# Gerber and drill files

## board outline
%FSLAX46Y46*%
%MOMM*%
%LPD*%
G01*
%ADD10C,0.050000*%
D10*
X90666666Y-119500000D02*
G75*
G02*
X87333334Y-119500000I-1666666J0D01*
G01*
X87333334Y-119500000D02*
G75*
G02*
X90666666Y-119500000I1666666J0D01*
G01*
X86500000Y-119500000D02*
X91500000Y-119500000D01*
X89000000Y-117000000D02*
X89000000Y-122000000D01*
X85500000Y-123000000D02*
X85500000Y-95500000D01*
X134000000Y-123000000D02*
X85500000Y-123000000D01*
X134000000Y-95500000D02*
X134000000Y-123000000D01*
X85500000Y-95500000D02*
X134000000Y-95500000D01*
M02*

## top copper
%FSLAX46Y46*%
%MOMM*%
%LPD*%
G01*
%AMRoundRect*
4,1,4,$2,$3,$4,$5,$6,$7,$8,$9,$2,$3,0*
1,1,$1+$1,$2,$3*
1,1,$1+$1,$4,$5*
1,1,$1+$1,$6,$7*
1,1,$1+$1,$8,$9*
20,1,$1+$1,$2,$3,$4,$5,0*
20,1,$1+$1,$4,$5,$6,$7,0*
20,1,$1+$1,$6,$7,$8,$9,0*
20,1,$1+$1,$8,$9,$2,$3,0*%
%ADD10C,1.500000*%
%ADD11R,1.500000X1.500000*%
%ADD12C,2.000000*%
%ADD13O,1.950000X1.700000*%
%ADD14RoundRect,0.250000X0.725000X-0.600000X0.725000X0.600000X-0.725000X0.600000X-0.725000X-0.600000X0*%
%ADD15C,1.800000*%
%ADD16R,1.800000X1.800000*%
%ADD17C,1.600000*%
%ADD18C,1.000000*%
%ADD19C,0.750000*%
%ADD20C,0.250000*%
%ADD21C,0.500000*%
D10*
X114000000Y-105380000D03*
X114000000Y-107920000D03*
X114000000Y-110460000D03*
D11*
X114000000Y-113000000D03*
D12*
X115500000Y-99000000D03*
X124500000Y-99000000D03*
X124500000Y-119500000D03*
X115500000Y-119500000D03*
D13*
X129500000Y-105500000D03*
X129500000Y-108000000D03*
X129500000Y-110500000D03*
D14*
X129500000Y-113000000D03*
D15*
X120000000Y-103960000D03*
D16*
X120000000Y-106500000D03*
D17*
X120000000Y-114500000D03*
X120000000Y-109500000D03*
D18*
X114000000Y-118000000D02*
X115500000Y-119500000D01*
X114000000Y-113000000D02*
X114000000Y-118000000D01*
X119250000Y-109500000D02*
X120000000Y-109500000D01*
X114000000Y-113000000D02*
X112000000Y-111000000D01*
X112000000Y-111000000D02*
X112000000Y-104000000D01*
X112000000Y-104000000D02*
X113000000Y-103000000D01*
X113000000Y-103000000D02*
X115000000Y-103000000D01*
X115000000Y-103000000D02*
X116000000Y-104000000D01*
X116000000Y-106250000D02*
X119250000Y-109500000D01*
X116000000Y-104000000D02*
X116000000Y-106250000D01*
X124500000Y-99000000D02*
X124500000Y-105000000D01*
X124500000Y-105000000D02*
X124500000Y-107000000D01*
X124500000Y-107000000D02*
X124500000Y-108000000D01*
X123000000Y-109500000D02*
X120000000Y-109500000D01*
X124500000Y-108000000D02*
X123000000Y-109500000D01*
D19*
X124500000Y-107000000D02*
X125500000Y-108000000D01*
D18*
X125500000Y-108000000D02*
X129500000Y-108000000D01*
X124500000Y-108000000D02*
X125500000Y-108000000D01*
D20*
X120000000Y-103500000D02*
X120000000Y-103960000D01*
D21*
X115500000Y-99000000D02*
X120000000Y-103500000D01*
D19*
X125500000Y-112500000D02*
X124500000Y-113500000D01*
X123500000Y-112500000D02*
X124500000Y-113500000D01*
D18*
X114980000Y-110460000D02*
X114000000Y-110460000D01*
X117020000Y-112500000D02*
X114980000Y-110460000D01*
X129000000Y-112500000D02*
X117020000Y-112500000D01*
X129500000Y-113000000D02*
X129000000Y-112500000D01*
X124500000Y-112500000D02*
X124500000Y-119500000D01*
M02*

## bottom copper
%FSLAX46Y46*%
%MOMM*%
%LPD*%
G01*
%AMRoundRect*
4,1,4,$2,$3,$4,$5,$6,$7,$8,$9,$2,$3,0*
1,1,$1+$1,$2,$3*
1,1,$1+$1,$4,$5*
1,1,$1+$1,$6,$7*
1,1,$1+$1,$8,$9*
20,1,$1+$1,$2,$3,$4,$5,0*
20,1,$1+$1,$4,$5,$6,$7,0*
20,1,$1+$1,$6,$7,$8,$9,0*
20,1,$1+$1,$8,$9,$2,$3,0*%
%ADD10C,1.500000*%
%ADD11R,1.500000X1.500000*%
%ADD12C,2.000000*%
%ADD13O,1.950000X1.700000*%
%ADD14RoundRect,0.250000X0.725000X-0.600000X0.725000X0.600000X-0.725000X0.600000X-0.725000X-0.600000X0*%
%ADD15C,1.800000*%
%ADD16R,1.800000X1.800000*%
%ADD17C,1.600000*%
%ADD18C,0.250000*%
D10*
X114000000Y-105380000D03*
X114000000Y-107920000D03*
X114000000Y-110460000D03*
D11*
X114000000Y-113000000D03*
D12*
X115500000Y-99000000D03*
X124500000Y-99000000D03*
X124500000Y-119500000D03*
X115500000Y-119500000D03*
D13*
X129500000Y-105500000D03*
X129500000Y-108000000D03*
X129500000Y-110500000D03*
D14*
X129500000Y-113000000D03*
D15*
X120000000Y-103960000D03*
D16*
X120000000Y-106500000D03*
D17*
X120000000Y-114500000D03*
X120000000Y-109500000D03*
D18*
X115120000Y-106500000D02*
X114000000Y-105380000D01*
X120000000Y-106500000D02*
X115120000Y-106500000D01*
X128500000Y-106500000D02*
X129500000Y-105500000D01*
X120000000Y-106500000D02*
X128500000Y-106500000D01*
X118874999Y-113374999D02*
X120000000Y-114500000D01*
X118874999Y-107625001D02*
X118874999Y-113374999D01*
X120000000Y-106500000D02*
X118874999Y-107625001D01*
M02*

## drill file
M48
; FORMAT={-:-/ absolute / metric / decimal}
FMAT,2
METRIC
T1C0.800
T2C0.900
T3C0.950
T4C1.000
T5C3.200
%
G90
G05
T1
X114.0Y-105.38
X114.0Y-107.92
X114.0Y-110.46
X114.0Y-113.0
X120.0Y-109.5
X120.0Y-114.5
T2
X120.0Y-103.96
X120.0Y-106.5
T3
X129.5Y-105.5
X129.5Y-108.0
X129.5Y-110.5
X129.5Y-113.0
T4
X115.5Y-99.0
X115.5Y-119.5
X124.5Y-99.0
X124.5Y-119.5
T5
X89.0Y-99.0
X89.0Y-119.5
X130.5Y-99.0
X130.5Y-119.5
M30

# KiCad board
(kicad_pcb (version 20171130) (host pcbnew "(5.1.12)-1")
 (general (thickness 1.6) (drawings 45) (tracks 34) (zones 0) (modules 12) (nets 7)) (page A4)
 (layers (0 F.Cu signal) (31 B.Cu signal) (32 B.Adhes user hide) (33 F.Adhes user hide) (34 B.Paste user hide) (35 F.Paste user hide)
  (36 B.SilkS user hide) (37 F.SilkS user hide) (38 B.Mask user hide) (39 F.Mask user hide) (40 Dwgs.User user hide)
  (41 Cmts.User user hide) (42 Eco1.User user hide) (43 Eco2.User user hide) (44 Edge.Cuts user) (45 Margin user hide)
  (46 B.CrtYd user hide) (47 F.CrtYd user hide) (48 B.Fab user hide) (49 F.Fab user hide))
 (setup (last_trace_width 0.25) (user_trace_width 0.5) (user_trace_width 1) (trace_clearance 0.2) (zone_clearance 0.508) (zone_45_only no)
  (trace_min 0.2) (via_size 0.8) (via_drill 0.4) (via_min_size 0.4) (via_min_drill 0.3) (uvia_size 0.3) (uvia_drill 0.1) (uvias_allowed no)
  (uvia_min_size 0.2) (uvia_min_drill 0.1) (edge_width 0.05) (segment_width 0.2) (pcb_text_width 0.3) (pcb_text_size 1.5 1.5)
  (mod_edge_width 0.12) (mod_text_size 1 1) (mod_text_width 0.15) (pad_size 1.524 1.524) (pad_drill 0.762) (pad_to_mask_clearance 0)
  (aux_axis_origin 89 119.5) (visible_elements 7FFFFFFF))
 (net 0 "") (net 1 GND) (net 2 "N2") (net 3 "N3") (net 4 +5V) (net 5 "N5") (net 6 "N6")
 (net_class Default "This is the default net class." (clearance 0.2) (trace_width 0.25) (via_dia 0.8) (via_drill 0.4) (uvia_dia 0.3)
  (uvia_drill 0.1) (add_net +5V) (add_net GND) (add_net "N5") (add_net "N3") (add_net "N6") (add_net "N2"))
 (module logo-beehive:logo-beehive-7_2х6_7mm (layer F.Cu) (at 98 119)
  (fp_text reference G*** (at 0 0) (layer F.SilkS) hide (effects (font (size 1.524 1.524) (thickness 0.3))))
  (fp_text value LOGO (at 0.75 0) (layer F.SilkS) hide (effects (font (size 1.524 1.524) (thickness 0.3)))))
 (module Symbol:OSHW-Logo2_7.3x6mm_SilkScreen (layer F.Cu) (at 106.5 119.5)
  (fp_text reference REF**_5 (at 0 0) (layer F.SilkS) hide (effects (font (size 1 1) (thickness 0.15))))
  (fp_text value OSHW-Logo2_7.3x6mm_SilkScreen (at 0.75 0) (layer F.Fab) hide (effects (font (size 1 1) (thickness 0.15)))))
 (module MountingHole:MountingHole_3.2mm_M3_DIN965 (layer F.Cu) (at 89 119.5 180)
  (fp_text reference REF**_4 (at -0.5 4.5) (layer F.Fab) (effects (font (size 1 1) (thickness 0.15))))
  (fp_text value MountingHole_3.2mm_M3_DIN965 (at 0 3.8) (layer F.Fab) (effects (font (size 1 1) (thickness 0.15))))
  (pad 1 np_thru_hole circle (at 0 0 180) (size 3.2 3.2) (drill 3.2) (layers *.Cu *.Mask)))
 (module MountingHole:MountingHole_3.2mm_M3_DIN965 (layer F.Cu) (at 89 99 90)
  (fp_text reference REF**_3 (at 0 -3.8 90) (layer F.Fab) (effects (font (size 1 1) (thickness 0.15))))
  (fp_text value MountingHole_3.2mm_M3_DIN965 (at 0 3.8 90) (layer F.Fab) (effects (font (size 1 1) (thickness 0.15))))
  (pad 1 np_thru_hole circle (at 0 0 90) (size 3.2 3.2) (drill 3.2) (layers *.Cu *.Mask)))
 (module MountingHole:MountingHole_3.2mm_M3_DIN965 (layer F.Cu) (at 130.5 119.5)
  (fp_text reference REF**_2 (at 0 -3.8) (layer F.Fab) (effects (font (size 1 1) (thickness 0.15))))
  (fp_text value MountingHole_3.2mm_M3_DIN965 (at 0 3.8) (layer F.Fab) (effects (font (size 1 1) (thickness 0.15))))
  (pad 1 np_thru_hole circle (at 0 0) (size 3.2 3.2) (drill 3.2) (layers *.Cu *.Mask)))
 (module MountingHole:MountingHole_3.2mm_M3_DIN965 (layer F.Cu) (at 130.5 99)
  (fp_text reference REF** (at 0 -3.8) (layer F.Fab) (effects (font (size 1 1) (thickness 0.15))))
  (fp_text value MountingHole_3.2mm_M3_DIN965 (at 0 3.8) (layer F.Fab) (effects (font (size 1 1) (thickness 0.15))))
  (pad 1 np_thru_hole circle (at 0 0) (size 3.2 3.2) (drill 3.2) (layers *.Cu *.Mask)))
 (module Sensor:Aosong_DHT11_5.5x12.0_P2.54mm (layer F.Cu) (at 114 113 180)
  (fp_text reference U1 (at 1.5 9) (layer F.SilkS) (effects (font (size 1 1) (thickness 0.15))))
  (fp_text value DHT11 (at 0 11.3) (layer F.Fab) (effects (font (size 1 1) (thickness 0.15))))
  (pad 4 thru_hole circle (at 0 7.62 180) (size 1.5 1.5) (drill 0.8) (layers *.Cu *.Mask) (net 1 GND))
  (pad 3 thru_hole circle (at 0 5.08 180) (size 1.5 1.5) (drill 0.8) (layers *.Cu *.Mask) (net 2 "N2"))
  (pad 2 thru_hole circle (at 0 2.54 180) (size 1.5 1.5) (drill 0.8) (layers *.Cu *.Mask) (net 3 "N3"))
  (pad 1 thru_hole rect (at 0 0 180) (size 1.5 1.5) (drill 0.8) (layers *.Cu *.Mask) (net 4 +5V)))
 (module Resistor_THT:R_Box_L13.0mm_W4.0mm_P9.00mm (layer F.Cu) (at 124.5 99 180)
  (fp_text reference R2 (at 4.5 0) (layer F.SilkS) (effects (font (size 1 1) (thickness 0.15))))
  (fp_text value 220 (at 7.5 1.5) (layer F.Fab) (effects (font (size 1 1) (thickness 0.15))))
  (pad 2 thru_hole circle (at 9 0 180) (size 2 2) (drill 1) (layers *.Cu *.Mask) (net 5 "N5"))
  (pad 1 thru_hole circle (at 0 0 180) (size 2 2) (drill 1) (layers *.Cu *.Mask) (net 4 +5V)))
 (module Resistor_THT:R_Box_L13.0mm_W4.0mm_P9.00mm (layer F.Cu) (at 115.5 119.5)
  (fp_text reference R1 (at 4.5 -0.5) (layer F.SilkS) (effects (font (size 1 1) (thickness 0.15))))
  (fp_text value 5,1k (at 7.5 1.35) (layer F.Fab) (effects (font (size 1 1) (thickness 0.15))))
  (pad 2 thru_hole circle (at 9 0) (size 2 2) (drill 1) (layers *.Cu *.Mask) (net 3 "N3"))
  (pad 1 thru_hole circle (at 0 0) (size 2 2) (drill 1) (layers *.Cu *.Mask) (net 4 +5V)))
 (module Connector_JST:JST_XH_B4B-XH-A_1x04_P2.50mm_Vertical (layer F.Cu) (at 129.5 113 90)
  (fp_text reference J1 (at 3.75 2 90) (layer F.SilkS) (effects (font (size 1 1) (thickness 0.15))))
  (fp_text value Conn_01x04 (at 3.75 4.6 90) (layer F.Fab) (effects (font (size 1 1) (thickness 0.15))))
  (pad 4 thru_hole oval (at 7.5 0 90) (size 1.7 1.95) (drill 0.95) (layers *.Cu *.Mask) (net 1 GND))
  (pad 3 thru_hole oval (at 5 0 90) (size 1.7 1.95) (drill 0.95) (layers *.Cu *.Mask) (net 4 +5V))
  (pad 2 thru_hole oval (at 2.5 0 90) (size 1.7 1.95) (drill 0.95) (layers *.Cu *.Mask) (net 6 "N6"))
  (pad 1 thru_hole roundrect (at 0 0 90) (size 1.7 1.95) (drill 0.95) (layers *.Cu *.Mask) (roundrect_rratio 0.1470588235294118)
   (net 3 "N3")))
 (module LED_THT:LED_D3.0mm (layer F.Cu) (at 120 106.5 90)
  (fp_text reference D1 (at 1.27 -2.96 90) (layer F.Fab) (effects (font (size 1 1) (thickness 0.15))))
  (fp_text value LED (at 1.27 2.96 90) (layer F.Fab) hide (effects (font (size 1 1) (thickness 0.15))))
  (pad 2 thru_hole circle (at 2.54 0 90) (size 1.8 1.8) (drill 0.9) (layers *.Cu *.Mask) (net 5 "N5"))
  (pad 1 thru_hole rect (at 0 0 90) (size 1.8 1.8) (drill 0.9) (layers *.Cu *.Mask) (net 1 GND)))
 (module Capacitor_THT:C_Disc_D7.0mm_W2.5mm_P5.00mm (layer F.Cu) (at 120 109.5 270)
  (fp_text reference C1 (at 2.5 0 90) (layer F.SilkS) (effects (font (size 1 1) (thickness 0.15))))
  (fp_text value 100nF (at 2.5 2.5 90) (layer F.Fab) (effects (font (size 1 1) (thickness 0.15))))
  (pad 2 thru_hole circle (at 5 0 270) (size 1.6 1.6) (drill 0.8) (layers *.Cu *.Mask) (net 1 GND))
  (pad 1 thru_hole circle (at 0 0 270) (size 1.6 1.6) (drill 0.8) (layers *.Cu *.Mask) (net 4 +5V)))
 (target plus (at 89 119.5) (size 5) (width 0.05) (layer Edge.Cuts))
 (gr_line (start 85.5 123) (end 85.5 95.5) (layer Edge.Cuts) (width 0.05))
 (gr_line (start 134 123) (end 85.5 123) (layer Edge.Cuts) (width 0.05))
 (gr_line (start 134 95.5) (end 134 123) (layer Edge.Cuts) (width 0.05))
 (gr_line (start 85.5 95.5) (end 134 95.5) (layer Edge.Cuts) (width 0.05))
 (segment (start 115.12 106.5) (end 114 105.38) (width 0.25) (layer B.Cu) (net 1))
 (segment (start 120 106.5) (end 115.12 106.5) (width 0.25) (layer B.Cu) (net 1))
 (segment (start 128.5 106.5) (end 129.5 105.5) (width 0.25) (layer B.Cu) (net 1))
 (segment (start 120 106.5) (end 128.5 106.5) (width 0.25) (layer B.Cu) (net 1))
 (segment (start 118.874999 113.374999) (end 120 114.5) (width 0.25) (layer B.Cu) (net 1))
 (segment (start 118.874999 107.625001) (end 118.874999 113.374999) (width 0.25) (layer B.Cu) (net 1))
 (segment (start 120 106.5) (end 118.874999 107.625001) (width 0.25) (layer B.Cu) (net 1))
 (segment (start 114 118) (end 115.5 119.5) (width 1) (layer F.Cu) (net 4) (status 20))
 (segment (start 114 113) (end 114 118) (width 1) (layer F.Cu) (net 4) (status 10))
 (segment (start 119.25 109.5) (end 120 109.5) (width 1) (layer F.Cu) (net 4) (status 30))
 (segment (start 114 113) (end 112 111) (width 1) (layer F.Cu) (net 4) (status 10))
 (segment (start 112 111) (end 112 104) (width 1) (layer F.Cu) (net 4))
 (segment (start 112 104) (end 113 103) (width 1) (layer F.Cu) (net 4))
 (segment (start 113 103) (end 115 103) (width 1) (layer F.Cu) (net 4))
 (segment (start 115 103) (end 116 104) (width 1) (layer F.Cu) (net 4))
 (segment (start 116 106.25) (end 119.25 109.5) (width 1) (layer F.Cu) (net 4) (status 20))
 (segment (start 116 104) (end 116 106.25) (width 1) (layer F.Cu) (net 4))
 (segment (start 124.5 99) (end 124.5 105) (width 1) (layer F.Cu) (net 4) (status 10))
 (segment (start 124.5 105) (end 124.5 107) (width 1) (layer F.Cu) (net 4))
 (segment (start 124.5 107) (end 124.5 108) (width 1) (layer F.Cu) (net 4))
 (segment (start 123 109.5) (end 120 109.5) (width 1) (layer F.Cu) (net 4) (status 20))
 (segment (start 124.5 108) (end 123 109.5) (width 1) (layer F.Cu) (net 4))
 (segment (start 124.5 107) (end 125.5 108) (width 0.75) (layer F.Cu) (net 4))
 (segment (start 125.5 108) (end 129.5 108) (width 1) (layer F.Cu) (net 4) (status 20))
 (segment (start 124.5 108) (end 125.5 108) (width 1) (layer F.Cu) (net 4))
 (segment (start 120 103.5) (end 120 103.96) (width 0.25) (layer F.Cu) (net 5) (status 30))
 (segment (start 115.5 99) (end 120 103.5) (width 0.5) (layer F.Cu) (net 5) (status 30))
 (segment (start 125.5 112.5) (end 124.5 113.5) (width 0.75) (layer F.Cu) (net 3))
 (segment (start 123.5 112.5) (end 124.5 113.5) (width 0.75) (layer F.Cu) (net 3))
 (segment (start 114.98 110.46) (end 114 110.46) (width 1) (layer F.Cu) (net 3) (status 20))
 (segment (start 117.02 112.5) (end 114.98 110.46) (width 1) (layer F.Cu) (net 3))
 (segment (start 129 112.5) (end 117.02 112.5) (width 1) (layer F.Cu) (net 3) (status 10))
 (segment (start 129.5 113) (end 129 112.5) (width 1) (layer F.Cu) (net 3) (status 30))
 (segment (start 124.5 112.5) (end 124.5 119.5) (width 1) (layer F.Cu) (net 3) (status 20)))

